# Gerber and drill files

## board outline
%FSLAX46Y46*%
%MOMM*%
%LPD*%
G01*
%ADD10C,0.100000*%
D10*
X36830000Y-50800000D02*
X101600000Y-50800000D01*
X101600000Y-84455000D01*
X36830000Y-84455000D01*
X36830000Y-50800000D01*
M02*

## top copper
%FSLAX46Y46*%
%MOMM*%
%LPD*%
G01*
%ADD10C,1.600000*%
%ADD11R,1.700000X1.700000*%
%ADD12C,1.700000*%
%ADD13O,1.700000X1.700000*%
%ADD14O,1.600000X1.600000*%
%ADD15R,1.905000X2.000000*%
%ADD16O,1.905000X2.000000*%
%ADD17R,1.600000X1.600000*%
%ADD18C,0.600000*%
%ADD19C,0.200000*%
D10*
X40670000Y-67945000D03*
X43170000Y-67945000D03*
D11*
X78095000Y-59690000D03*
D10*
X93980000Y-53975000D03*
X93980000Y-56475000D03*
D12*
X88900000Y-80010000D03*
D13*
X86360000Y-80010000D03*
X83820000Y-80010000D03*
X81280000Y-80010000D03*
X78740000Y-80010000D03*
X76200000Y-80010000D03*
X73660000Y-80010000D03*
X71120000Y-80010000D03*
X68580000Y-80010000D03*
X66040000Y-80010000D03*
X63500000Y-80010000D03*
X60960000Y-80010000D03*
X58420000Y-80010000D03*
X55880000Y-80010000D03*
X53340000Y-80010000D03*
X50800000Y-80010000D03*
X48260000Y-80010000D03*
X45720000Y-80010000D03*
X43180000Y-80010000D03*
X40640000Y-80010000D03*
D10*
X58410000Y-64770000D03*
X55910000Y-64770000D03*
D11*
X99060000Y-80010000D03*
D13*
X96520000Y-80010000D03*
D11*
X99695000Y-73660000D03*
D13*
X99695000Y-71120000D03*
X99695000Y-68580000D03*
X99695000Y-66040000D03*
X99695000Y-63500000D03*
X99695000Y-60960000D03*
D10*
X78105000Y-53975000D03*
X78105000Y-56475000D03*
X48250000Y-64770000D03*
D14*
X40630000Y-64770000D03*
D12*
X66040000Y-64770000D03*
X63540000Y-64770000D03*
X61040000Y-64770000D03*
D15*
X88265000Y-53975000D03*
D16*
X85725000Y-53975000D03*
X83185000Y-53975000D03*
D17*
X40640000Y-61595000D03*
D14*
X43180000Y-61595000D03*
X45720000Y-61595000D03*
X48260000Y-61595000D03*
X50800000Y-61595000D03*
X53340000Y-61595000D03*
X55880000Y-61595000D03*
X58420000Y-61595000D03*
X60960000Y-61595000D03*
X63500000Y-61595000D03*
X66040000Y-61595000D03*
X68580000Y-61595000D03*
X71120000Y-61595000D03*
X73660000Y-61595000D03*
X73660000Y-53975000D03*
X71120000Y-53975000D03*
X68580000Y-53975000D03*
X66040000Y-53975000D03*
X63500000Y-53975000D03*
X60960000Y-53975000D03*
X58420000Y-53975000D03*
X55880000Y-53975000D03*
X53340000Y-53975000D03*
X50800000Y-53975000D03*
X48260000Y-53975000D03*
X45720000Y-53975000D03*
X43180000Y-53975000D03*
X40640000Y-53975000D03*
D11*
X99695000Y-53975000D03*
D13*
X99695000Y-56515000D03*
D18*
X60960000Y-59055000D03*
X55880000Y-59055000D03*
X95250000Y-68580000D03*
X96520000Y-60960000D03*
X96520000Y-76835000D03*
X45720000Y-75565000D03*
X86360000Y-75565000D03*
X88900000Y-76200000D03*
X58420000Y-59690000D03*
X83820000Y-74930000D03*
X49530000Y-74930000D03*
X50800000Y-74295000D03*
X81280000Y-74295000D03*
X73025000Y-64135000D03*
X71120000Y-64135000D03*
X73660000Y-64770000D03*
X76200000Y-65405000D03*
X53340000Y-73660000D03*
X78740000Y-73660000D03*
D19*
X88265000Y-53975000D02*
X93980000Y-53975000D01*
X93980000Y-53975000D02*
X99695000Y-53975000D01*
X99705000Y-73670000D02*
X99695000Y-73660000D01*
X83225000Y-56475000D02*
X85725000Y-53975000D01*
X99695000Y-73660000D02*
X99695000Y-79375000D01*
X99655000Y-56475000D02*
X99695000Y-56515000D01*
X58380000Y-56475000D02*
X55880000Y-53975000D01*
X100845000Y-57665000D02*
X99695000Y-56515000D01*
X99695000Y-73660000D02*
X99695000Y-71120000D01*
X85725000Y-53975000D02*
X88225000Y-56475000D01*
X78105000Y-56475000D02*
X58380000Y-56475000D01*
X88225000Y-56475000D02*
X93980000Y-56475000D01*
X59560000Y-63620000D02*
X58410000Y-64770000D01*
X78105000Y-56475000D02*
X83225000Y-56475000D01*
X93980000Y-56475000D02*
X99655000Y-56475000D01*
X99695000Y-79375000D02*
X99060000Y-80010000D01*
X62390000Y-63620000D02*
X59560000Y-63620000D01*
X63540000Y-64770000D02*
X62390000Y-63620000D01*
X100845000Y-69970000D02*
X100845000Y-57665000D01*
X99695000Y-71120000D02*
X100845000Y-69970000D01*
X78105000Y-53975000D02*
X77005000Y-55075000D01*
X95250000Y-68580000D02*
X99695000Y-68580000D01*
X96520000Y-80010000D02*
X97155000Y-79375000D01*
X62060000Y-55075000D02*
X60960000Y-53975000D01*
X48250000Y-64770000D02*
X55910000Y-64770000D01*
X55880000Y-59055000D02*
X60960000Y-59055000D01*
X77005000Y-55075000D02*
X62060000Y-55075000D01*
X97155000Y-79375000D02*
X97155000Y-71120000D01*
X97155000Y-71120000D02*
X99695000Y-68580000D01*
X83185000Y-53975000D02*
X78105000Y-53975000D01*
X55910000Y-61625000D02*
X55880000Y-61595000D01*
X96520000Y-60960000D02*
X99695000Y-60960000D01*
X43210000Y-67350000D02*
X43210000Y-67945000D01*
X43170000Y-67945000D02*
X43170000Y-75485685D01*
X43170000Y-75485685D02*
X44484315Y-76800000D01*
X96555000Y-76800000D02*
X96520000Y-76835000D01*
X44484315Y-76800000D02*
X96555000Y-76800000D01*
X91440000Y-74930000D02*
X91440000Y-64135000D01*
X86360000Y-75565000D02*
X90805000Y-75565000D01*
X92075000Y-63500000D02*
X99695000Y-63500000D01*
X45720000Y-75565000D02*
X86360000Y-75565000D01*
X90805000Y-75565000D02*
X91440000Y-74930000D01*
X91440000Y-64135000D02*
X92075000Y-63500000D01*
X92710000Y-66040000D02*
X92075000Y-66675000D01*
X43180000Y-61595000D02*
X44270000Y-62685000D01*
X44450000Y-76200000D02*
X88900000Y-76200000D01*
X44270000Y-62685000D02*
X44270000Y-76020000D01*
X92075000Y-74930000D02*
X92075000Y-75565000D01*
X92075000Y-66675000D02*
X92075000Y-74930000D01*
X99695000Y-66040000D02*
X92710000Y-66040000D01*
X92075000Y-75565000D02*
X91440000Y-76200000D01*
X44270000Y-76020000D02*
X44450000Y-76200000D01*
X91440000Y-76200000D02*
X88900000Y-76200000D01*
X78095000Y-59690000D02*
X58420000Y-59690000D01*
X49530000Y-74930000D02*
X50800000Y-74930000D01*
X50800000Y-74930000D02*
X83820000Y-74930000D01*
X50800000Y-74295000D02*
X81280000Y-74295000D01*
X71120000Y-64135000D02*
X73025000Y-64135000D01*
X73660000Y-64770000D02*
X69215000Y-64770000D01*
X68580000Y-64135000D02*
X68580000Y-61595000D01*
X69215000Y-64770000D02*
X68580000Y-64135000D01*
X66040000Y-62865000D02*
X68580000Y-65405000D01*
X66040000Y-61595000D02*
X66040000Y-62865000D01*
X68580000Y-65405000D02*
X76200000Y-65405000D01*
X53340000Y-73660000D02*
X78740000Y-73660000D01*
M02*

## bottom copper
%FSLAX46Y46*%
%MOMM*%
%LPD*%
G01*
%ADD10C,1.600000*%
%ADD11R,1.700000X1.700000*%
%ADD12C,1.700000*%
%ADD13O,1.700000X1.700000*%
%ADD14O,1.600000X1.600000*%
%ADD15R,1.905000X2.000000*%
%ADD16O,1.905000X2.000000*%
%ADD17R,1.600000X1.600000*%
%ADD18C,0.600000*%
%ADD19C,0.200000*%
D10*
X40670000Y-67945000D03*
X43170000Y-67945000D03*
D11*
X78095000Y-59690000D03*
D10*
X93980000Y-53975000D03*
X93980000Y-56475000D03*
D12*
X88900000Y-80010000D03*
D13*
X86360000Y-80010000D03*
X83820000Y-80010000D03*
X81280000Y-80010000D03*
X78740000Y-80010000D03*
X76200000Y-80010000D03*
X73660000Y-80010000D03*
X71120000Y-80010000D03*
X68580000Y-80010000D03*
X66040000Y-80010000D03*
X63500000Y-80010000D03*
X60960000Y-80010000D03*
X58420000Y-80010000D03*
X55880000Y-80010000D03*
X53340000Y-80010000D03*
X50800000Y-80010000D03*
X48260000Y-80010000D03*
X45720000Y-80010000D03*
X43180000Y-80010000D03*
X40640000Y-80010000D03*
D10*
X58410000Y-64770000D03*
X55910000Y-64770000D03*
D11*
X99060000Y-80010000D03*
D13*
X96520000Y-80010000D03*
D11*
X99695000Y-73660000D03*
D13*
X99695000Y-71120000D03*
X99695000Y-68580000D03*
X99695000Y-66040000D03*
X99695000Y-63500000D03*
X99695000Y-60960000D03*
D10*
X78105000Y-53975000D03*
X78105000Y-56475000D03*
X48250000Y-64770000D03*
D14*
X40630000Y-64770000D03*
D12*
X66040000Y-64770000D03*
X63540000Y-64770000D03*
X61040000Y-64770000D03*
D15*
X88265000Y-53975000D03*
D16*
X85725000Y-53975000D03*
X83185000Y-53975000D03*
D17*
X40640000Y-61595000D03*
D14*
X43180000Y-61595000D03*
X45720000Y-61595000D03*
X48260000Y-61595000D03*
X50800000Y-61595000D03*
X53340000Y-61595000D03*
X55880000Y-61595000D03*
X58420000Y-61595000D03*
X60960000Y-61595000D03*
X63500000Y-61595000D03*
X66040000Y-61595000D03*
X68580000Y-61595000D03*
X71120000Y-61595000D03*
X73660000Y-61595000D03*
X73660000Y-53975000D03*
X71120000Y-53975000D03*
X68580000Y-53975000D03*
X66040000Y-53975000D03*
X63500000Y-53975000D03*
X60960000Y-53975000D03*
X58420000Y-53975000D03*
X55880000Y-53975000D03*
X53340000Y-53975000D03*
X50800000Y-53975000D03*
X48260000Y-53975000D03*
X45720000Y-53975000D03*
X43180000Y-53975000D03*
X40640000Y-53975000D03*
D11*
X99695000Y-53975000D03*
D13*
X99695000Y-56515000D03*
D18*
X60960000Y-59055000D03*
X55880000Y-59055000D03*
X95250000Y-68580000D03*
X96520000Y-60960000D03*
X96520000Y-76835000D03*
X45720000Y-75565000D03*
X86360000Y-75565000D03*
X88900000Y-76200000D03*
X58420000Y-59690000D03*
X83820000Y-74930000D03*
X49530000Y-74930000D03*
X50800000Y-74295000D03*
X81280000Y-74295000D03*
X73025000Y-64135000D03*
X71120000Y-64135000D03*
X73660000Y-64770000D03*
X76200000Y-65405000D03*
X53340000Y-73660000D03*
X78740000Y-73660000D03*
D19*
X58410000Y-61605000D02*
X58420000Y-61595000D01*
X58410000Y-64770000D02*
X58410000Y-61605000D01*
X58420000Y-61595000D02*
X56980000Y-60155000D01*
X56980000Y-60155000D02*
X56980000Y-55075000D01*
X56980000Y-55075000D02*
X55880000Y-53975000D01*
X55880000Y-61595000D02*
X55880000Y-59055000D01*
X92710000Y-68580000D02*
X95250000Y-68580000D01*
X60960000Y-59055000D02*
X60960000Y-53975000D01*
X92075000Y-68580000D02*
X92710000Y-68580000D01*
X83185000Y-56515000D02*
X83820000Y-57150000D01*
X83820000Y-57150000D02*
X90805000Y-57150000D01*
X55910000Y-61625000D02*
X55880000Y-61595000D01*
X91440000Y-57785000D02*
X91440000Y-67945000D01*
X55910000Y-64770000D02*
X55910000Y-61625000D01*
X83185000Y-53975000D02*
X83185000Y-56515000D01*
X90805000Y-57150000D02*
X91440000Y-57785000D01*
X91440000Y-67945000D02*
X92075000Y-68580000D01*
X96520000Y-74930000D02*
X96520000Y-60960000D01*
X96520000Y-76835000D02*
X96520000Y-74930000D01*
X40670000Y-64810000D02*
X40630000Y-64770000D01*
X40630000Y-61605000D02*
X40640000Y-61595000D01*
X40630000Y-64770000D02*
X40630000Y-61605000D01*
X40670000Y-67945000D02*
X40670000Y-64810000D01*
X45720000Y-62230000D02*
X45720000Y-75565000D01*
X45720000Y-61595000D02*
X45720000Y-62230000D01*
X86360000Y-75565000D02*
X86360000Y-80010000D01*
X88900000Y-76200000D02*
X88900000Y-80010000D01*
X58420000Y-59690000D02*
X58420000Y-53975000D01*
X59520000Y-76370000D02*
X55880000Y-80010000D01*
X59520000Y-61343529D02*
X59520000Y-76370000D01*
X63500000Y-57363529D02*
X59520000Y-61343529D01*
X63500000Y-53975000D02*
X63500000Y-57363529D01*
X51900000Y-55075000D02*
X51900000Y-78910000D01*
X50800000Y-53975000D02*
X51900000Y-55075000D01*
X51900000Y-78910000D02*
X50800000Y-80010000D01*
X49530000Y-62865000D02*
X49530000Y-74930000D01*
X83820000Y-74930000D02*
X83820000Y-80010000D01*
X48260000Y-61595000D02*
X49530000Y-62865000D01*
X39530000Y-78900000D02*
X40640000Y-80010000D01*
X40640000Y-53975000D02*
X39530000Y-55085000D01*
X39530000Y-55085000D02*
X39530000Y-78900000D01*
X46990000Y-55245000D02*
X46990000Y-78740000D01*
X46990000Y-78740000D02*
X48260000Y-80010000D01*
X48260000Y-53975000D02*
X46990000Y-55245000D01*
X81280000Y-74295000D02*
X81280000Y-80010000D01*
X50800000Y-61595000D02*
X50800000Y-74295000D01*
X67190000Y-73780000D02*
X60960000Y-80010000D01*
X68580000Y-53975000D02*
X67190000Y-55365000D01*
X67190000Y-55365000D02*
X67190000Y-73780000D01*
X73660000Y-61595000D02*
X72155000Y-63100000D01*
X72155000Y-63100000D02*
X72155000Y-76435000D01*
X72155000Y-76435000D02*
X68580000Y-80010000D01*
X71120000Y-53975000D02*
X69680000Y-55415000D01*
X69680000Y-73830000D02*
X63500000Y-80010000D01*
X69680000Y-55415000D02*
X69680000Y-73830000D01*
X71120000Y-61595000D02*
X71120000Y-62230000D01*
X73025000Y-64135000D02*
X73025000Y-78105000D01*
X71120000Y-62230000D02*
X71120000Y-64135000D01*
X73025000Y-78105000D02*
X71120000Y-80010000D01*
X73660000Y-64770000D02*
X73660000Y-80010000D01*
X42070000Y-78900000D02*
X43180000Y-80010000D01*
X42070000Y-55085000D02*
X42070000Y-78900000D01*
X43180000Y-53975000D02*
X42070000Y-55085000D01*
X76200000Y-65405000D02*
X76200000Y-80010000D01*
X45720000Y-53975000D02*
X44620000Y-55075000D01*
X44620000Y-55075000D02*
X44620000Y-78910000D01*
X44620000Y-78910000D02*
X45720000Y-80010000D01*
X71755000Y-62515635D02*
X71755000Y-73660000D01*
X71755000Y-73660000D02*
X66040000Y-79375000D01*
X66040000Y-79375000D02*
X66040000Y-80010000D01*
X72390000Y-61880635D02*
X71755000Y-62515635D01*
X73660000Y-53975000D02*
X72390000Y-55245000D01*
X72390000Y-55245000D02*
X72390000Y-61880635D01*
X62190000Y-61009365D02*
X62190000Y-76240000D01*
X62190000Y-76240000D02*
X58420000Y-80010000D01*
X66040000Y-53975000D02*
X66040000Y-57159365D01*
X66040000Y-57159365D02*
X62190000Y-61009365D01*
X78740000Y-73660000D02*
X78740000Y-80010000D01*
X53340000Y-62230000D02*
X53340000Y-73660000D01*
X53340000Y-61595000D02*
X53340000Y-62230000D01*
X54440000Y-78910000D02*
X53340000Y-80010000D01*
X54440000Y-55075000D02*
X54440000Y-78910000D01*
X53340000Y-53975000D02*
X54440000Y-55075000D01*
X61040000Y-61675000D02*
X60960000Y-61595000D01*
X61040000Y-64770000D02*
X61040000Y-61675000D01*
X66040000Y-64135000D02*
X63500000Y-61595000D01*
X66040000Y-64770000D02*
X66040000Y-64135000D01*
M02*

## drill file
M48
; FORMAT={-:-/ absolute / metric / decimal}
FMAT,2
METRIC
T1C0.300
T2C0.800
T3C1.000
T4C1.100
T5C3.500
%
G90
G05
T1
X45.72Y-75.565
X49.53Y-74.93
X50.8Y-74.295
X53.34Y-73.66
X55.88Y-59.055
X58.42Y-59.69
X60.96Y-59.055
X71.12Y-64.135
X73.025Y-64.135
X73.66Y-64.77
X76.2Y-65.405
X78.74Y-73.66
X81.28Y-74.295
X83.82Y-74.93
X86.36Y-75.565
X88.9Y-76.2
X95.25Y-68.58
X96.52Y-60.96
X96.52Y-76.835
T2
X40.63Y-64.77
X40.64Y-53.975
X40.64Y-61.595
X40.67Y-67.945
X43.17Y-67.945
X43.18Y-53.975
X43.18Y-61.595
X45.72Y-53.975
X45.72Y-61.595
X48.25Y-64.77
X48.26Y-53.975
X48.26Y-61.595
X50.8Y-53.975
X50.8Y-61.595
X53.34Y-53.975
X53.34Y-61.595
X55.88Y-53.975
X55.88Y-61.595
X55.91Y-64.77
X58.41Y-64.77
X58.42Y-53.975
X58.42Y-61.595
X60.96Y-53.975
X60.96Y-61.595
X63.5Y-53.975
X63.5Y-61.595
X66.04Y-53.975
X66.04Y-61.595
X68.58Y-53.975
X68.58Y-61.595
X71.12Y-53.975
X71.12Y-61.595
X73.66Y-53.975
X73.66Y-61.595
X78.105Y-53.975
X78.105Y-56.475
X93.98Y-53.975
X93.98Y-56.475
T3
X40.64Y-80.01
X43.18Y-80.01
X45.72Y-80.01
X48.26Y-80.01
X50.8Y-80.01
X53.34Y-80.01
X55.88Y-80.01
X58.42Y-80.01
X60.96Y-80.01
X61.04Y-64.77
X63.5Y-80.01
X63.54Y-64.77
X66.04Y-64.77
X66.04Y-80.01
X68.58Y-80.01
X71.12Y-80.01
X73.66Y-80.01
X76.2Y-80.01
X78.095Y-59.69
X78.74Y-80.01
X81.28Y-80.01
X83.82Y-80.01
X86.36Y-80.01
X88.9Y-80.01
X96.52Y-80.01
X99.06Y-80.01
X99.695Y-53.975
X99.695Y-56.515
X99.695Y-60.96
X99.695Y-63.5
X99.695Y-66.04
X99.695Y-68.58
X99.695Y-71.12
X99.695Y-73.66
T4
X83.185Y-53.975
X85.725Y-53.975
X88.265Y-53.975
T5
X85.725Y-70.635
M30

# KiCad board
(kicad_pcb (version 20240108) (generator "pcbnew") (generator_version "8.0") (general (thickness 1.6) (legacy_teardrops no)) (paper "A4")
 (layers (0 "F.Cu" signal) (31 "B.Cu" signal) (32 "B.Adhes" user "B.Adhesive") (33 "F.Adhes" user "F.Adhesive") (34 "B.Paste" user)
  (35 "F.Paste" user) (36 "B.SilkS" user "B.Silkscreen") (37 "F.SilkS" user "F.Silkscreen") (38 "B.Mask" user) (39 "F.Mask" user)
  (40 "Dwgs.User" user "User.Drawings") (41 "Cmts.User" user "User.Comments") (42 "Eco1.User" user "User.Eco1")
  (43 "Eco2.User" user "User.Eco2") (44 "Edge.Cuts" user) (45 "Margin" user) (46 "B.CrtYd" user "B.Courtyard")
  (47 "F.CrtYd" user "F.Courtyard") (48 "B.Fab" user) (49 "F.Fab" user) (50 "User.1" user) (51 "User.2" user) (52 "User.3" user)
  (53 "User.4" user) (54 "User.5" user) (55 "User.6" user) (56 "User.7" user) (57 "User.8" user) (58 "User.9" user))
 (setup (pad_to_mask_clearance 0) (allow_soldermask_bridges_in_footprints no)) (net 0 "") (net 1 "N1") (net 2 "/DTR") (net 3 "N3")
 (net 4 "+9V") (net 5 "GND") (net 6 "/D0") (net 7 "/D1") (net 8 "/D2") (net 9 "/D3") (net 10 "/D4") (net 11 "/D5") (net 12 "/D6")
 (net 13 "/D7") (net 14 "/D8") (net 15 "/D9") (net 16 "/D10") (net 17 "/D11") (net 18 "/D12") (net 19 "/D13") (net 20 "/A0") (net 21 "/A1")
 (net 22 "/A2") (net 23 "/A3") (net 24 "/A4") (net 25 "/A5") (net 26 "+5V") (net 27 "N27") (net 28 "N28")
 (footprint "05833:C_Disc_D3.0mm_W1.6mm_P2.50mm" (layer "F.Cu") (at 40.67 67.945)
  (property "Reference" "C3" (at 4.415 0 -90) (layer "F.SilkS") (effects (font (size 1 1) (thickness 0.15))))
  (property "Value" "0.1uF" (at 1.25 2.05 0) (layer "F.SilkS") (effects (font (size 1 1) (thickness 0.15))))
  (pad "1" thru_hole circle (at 0 0) (size 1.6 1.6) (drill 0.8) (layers "*.Cu" "*.Mask") (remove_unused_layers no) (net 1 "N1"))
  (pad "2" thru_hole circle (at 2.5 0) (size 1.6 1.6) (drill 0.8) (layers "*.Cu" "*.Mask") (remove_unused_layers no) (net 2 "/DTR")))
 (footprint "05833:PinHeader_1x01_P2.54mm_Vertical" (layer "F.Cu") (at 78.095 59.69)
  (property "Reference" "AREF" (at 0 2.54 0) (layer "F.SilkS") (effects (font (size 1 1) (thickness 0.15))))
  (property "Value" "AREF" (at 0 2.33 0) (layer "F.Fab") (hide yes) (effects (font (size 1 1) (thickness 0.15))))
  (pad "1" thru_hole rect (at 0 0) (size 1.7 1.7) (drill 1) (layers "*.Cu" "*.Mask") (remove_unused_layers no) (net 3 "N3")))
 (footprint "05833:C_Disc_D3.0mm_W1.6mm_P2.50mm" (layer "F.Cu") (at 93.98 53.975 -90)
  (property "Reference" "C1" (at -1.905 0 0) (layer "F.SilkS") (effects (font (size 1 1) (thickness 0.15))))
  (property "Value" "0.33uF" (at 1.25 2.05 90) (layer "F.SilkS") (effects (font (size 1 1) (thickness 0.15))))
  (pad "1" thru_hole circle (at 0 0 270) (size 1.6 1.6) (drill 0.8) (layers "*.Cu" "*.Mask") (remove_unused_layers no) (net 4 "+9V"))
  (pad "2" thru_hole circle (at 2.5 0 270) (size 1.6 1.6) (drill 0.8) (layers "*.Cu" "*.Mask") (remove_unused_layers no) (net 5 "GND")))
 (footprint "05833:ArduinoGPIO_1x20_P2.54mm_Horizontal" (layer "F.Cu") (at 88.9 80.01 -90)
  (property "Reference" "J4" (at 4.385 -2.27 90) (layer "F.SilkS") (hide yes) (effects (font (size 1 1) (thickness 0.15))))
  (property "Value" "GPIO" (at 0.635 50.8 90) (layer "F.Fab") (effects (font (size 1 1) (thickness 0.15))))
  (pad "1" thru_hole circle (at 0 0 270) (size 1.7 1.7) (drill 1) (layers "*.Cu" "*.Mask") (remove_unused_layers no) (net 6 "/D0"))
  (pad "2" thru_hole oval (at 0 2.54 270) (size 1.7 1.7) (drill 1) (layers "*.Cu" "*.Mask") (remove_unused_layers no) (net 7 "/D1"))
  (pad "3" thru_hole oval (at 0 5.08 270) (size 1.7 1.7) (drill 1) (layers "*.Cu" "*.Mask") (remove_unused_layers no) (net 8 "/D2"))
  (pad "4" thru_hole oval (at 0 7.62 270) (size 1.7 1.7) (drill 1) (layers "*.Cu" "*.Mask") (remove_unused_layers no) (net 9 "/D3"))
  (pad "5" thru_hole oval (at 0 10.16 270) (size 1.7 1.7) (drill 1) (layers "*.Cu" "*.Mask") (remove_unused_layers no) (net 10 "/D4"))
  (pad "6" thru_hole oval (at 0 12.7 270) (size 1.7 1.7) (drill 1) (layers "*.Cu" "*.Mask") (remove_unused_layers no) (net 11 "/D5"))
  (pad "7" thru_hole oval (at 0 15.24 270) (size 1.7 1.7) (drill 1) (layers "*.Cu" "*.Mask") (remove_unused_layers no) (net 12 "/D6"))
  (pad "8" thru_hole oval (at 0 17.78 270) (size 1.7 1.7) (drill 1) (layers "*.Cu" "*.Mask") (remove_unused_layers no) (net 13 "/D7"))
  (pad "9" thru_hole oval (at 0 20.32 270) (size 1.7 1.7) (drill 1) (layers "*.Cu" "*.Mask") (remove_unused_layers no) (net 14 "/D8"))
  (pad "10" thru_hole oval (at 0 22.86 270) (size 1.7 1.7) (drill 1) (layers "*.Cu" "*.Mask") (remove_unused_layers no) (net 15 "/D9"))
  (pad "11" thru_hole oval (at 0 25.4 270) (size 1.7 1.7) (drill 1) (layers "*.Cu" "*.Mask") (remove_unused_layers no) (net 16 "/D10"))
  (pad "12" thru_hole oval (at 0 27.94 270) (size 1.7 1.7) (drill 1) (layers "*.Cu" "*.Mask") (remove_unused_layers no) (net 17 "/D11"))
  (pad "13" thru_hole oval (at 0 30.48 270) (size 1.7 1.7) (drill 1) (layers "*.Cu" "*.Mask") (remove_unused_layers no) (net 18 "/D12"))
  (pad "14" thru_hole oval (at 0 33.02 270) (size 1.7 1.7) (drill 1) (layers "*.Cu" "*.Mask") (remove_unused_layers no) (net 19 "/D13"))
  (pad "15" thru_hole oval (at 0 35.56 270) (size 1.7 1.7) (drill 1) (layers "*.Cu" "*.Mask") (remove_unused_layers no) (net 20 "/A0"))
  (pad "16" thru_hole oval (at 0 38.1 270) (size 1.7 1.7) (drill 1) (layers "*.Cu" "*.Mask") (remove_unused_layers no) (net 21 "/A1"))
  (pad "17" thru_hole oval (at 0 40.64 270) (size 1.7 1.7) (drill 1) (layers "*.Cu" "*.Mask") (remove_unused_layers no) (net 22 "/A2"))
  (pad "18" thru_hole oval (at 0 43.18 270) (size 1.7 1.7) (drill 1) (layers "*.Cu" "*.Mask") (remove_unused_layers no) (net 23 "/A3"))
  (pad "19" thru_hole oval (at 0 45.72 270) (size 1.7 1.7) (drill 1) (layers "*.Cu" "*.Mask") (remove_unused_layers no) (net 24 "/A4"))
  (pad "20" thru_hole oval (at 0 48.26 270) (size 1.7 1.7) (drill 1) (layers "*.Cu" "*.Mask") (remove_unused_layers no) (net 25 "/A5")))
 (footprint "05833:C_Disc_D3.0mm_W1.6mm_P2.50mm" (layer "F.Cu") (at 58.41 64.77 180)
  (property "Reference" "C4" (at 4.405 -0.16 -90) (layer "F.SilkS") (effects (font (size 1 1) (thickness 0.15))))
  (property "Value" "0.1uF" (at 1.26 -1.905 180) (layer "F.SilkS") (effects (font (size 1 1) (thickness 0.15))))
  (pad "1" thru_hole circle (at 0 0 180) (size 1.6 1.6) (drill 0.8) (layers "*.Cu" "*.Mask") (remove_unused_layers no) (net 5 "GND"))
  (pad "2" thru_hole circle (at 2.5 0 180) (size 1.6 1.6) (drill 0.8) (layers "*.Cu" "*.Mask") (remove_unused_layers no) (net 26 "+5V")))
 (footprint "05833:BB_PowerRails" (layer "F.Cu") (at 99.06 80.01 -90)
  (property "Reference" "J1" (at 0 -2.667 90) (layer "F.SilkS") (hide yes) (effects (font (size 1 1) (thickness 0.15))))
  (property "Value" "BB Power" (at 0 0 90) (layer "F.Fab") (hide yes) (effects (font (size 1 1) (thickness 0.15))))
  (pad "1" thru_hole rect (at 0 0 270) (size 1.7 1.7) (drill 1) (layers "*.Cu" "*.Mask") (remove_unused_layers no) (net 5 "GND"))
  (pad "2" thru_hole oval (at 0 2.54 270) (size 1.7 1.7) (drill 1) (layers "*.Cu" "*.Mask") (remove_unused_layers no) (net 26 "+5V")))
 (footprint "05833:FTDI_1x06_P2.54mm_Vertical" (layer "F.Cu") (at 99.695 73.66 180)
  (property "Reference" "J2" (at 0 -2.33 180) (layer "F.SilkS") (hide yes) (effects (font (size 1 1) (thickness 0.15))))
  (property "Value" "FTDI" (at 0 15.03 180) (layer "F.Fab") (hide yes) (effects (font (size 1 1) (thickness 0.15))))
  (pad "1" thru_hole rect (at 0 0 180) (size 1.7 1.7) (drill 1) (layers "*.Cu" "*.Mask") (remove_unused_layers no) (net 5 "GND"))
  (pad "2" thru_hole oval (at 0 2.54 180) (size 1.7 1.7) (drill 1) (layers "*.Cu" "*.Mask") (remove_unused_layers no) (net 5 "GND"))
  (pad "3" thru_hole oval (at 0 5.08 180) (size 1.7 1.7) (drill 1) (layers "*.Cu" "*.Mask") (remove_unused_layers no) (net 26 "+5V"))
  (pad "4" thru_hole oval (at 0 7.62 180) (size 1.7 1.7) (drill 1) (layers "*.Cu" "*.Mask") (remove_unused_layers no) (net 6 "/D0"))
  (pad "5" thru_hole oval (at 0 10.16 180) (size 1.7 1.7) (drill 1) (layers "*.Cu" "*.Mask") (remove_unused_layers no) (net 7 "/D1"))
  (pad "6" thru_hole oval (at 0 12.7 180) (size 1.7 1.7) (drill 1) (layers "*.Cu" "*.Mask") (remove_unused_layers no) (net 2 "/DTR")))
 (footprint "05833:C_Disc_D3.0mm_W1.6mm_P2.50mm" (layer "F.Cu") (at 78.105 53.975 -90)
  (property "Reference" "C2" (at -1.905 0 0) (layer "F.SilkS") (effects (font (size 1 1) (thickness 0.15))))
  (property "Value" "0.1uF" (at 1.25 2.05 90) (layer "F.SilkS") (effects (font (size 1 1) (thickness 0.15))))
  (pad "1" thru_hole circle (at 0 0 270) (size 1.6 1.6) (drill 0.8) (layers "*.Cu" "*.Mask") (remove_unused_layers no) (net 26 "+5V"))
  (pad "2" thru_hole circle (at 2.5 0 270) (size 1.6 1.6) (drill 0.8) (layers "*.Cu" "*.Mask") (remove_unused_layers no) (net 5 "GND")))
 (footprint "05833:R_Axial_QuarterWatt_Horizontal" (layer "F.Cu") (at 48.25 64.77 180)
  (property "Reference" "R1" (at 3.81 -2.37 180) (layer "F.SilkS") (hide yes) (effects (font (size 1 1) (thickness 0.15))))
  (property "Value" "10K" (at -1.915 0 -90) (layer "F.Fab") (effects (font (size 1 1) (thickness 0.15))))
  (pad "1" thru_hole circle (at 0 0 180) (size 1.6 1.6) (drill 0.8) (layers "*.Cu" "*.Mask") (remove_unused_layers no) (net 26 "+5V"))
  (pad "2" thru_hole oval (at 7.62 0 180) (size 1.6 1.6) (drill 0.8) (layers "*.Cu" "*.Mask") (remove_unused_layers no) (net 1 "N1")))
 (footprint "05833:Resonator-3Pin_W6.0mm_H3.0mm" (layer "F.Cu") (at 66.04 64.77 180)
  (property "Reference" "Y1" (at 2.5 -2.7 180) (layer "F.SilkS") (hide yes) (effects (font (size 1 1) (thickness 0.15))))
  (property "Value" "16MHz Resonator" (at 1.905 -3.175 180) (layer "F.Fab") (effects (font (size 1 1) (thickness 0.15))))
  (pad "1" thru_hole circle (at 0 0 180) (size 1.7 1.7) (drill 1) (layers "*.Cu" "*.Mask") (remove_unused_layers no) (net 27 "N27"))
  (pad "2" thru_hole circle (at 2.5 0 180) (size 1.7 1.7) (drill 1) (layers "*.Cu" "*.Mask") (remove_unused_layers no) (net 5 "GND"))
  (pad "3" thru_hole circle (at 5 0 180) (size 1.7 1.7) (drill 1) (layers "*.Cu" "*.Mask") (remove_unused_layers no) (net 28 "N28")))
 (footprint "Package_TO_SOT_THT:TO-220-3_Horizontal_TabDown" (layer "F.Cu") (at 88.265 53.975 180)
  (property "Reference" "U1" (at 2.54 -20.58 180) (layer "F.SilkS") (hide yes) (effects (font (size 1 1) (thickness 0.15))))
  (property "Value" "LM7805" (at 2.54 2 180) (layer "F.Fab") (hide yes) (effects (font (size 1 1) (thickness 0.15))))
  (pad "" np_thru_hole oval (at 2.54 -16.66 180) (size 3.5 3.5) (drill 3.5) (layers "*.Cu" "*.Mask"))
  (pad "1" thru_hole rect (at 0 0 180) (size 1.905 2) (drill 1.1) (layers "*.Cu" "*.Mask") (remove_unused_layers no) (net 4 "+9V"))
  (pad "2" thru_hole oval (at 2.54 0 180) (size 1.905 2) (drill 1.1) (layers "*.Cu" "*.Mask") (remove_unused_layers no) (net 5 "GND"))
  (pad "3" thru_hole oval (at 5.08 0 180) (size 1.905 2) (drill 1.1) (layers "*.Cu" "*.Mask") (remove_unused_layers no) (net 26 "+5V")))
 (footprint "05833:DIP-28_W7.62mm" (layer "F.Cu") (at 40.64 61.595 90)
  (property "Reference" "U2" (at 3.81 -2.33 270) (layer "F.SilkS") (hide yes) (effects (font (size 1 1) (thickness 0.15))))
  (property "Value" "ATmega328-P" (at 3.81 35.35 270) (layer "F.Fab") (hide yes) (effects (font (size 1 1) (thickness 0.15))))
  (pad "1" thru_hole rect (at 0 0 90) (size 1.6 1.6) (drill 0.8) (layers "*.Cu" "*.Mask") (remove_unused_layers no) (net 1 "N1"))
  (pad "2" thru_hole oval (at 0 2.54 90) (size 1.6 1.6) (drill 0.8) (layers "*.Cu" "*.Mask") (remove_unused_layers no) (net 6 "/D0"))
  (pad "3" thru_hole oval (at 0 5.08 90) (size 1.6 1.6) (drill 0.8) (layers "*.Cu" "*.Mask") (remove_unused_layers no) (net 7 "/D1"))
  (pad "4" thru_hole oval (at 0 7.62 90) (size 1.6 1.6) (drill 0.8) (layers "*.Cu" "*.Mask") (remove_unused_layers no) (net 8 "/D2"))
  (pad "5" thru_hole oval (at 0 10.16 90) (size 1.6 1.6) (drill 0.8) (layers "*.Cu" "*.Mask") (remove_unused_layers no) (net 9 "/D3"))
  (pad "6" thru_hole oval (at 0 12.7 90) (size 1.6 1.6) (drill 0.8) (layers "*.Cu" "*.Mask") (remove_unused_layers no) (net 10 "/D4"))
  (pad "7" thru_hole oval (at 0 15.24 90) (size 1.6 1.6) (drill 0.8) (layers "*.Cu" "*.Mask") (remove_unused_layers no) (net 26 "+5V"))
  (pad "8" thru_hole oval (at 0 17.78 90) (size 1.6 1.6) (drill 0.8) (layers "*.Cu" "*.Mask") (remove_unused_layers no) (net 5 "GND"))
  (pad "9" thru_hole oval (at 0 20.32 90) (size 1.6 1.6) (drill 0.8) (layers "*.Cu" "*.Mask") (remove_unused_layers no) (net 28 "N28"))
  (pad "10" thru_hole oval (at 0 22.86 90) (size 1.6 1.6) (drill 0.8) (layers "*.Cu" "*.Mask") (remove_unused_layers no) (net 27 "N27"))
  (pad "11" thru_hole oval (at 0 25.4 90) (size 1.6 1.6) (drill 0.8) (layers "*.Cu" "*.Mask") (remove_unused_layers no) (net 11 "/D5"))
  (pad "12" thru_hole oval (at 0 27.94 90) (size 1.6 1.6) (drill 0.8) (layers "*.Cu" "*.Mask") (remove_unused_layers no) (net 12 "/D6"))
  (pad "13" thru_hole oval (at 0 30.48 90) (size 1.6 1.6) (drill 0.8) (layers "*.Cu" "*.Mask") (remove_unused_layers no) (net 13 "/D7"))
  (pad "14" thru_hole oval (at 0 33.02 90) (size 1.6 1.6) (drill 0.8) (layers "*.Cu" "*.Mask") (remove_unused_layers no) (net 14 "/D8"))
  (pad "15" thru_hole oval (at 7.62 33.02 90) (size 1.6 1.6) (drill 0.8) (layers "*.Cu" "*.Mask") (remove_unused_layers no) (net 15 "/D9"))
  (pad "16" thru_hole oval (at 7.62 30.48 90) (size 1.6 1.6) (drill 0.8) (layers "*.Cu" "*.Mask") (remove_unused_layers no) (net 16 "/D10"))
  (pad "17" thru_hole oval (at 7.62 27.94 90) (size 1.6 1.6) (drill 0.8) (layers "*.Cu" "*.Mask") (remove_unused_layers no) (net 17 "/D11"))
  (pad "18" thru_hole oval (at 7.62 25.4 90) (size 1.6 1.6) (drill 0.8) (layers "*.Cu" "*.Mask") (remove_unused_layers no) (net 18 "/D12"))
  (pad "19" thru_hole oval (at 7.62 22.86 90) (size 1.6 1.6) (drill 0.8) (layers "*.Cu" "*.Mask") (remove_unused_layers no) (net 19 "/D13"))
  (pad "20" thru_hole oval (at 7.62 20.32 90) (size 1.6 1.6) (drill 0.8) (layers "*.Cu" "*.Mask") (remove_unused_layers no) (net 26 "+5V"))
  (pad "21" thru_hole oval (at 7.62 17.78 90) (size 1.6 1.6) (drill 0.8) (layers "*.Cu" "*.Mask") (remove_unused_layers no) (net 3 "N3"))
  (pad "22" thru_hole oval (at 7.62 15.24 90) (size 1.6 1.6) (drill 0.8) (layers "*.Cu" "*.Mask") (remove_unused_layers no) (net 5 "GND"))
  (pad "23" thru_hole oval (at 7.62 12.7 90) (size 1.6 1.6) (drill 0.8) (layers "*.Cu" "*.Mask") (remove_unused_layers no) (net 20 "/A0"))
  (pad "24" thru_hole oval (at 7.62 10.16 90) (size 1.6 1.6) (drill 0.8) (layers "*.Cu" "*.Mask") (remove_unused_layers no) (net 21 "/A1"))
  (pad "25" thru_hole oval (at 7.62 7.62 90) (size 1.6 1.6) (drill 0.8) (layers "*.Cu" "*.Mask") (remove_unused_layers no) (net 22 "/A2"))
  (pad "26" thru_hole oval (at 7.62 5.08 90) (size 1.6 1.6) (drill 0.8) (layers "*.Cu" "*.Mask") (remove_unused_layers no) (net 23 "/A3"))
  (pad "27" thru_hole oval (at 7.62 2.54 90) (size 1.6 1.6) (drill 0.8) (layers "*.Cu" "*.Mask") (remove_unused_layers no) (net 24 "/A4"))
  (pad "28" thru_hole oval (at 7.62 0 90) (size 1.6 1.6) (drill 0.8) (layers "*.Cu" "*.Mask") (remove_unused_layers no) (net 25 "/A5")))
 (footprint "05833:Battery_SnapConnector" (layer "F.Cu") (at 99.695 53.975)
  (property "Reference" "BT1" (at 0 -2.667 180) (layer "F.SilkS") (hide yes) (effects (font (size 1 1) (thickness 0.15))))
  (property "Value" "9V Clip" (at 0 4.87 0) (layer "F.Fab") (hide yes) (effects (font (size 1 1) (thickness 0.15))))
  (pad "1" thru_hole rect (at 0 0) (size 1.7 1.7) (drill 1) (layers "*.Cu" "*.Mask") (remove_unused_layers no) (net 4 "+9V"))
  (pad "2" thru_hole oval (at 0 2.54) (size 1.7 1.7) (drill 1) (layers "*.Cu" "*.Mask") (remove_unused_layers no) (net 5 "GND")))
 (gr_rect (start 36.83 50.8) (end 101.6 84.455) (stroke (width 0.1) (type default)) (fill none) (layer "Edge.Cuts"))
 (segment (start 88.265 53.975) (end 93.98 53.975) (width 0.2) (layer "F.Cu") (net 4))
 (segment (start 93.98 53.975) (end 99.695 53.975) (width 0.2) (layer "F.Cu") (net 4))
 (segment (start 99.705 73.67) (end 99.695 73.66) (width 0.2) (layer "F.Cu") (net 5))
 (segment (start 83.225 56.475) (end 85.725 53.975) (width 0.2) (layer "F.Cu") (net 5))
 (segment (start 99.695 73.66) (end 99.695 79.375) (width 0.2) (layer "F.Cu") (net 5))
 (segment (start 99.655 56.475) (end 99.695 56.515) (width 0.2) (layer "F.Cu") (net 5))
 (segment (start 58.38 56.475) (end 55.88 53.975) (width 0.2) (layer "F.Cu") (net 5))
 (segment (start 100.845 57.665) (end 99.695 56.515) (width 0.2) (layer "F.Cu") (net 5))
 (segment (start 99.695 73.66) (end 99.695 71.12) (width 0.2) (layer "F.Cu") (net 5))
 (segment (start 85.725 53.975) (end 88.225 56.475) (width 0.2) (layer "F.Cu") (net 5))
 (segment (start 78.105 56.475) (end 58.38 56.475) (width 0.2) (layer "F.Cu") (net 5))
 (segment (start 88.225 56.475) (end 93.98 56.475) (width 0.2) (layer "F.Cu") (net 5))
 (segment (start 59.56 63.62) (end 58.41 64.77) (width 0.2) (layer "F.Cu") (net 5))
 (segment (start 78.105 56.475) (end 83.225 56.475) (width 0.2) (layer "F.Cu") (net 5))
 (segment (start 93.98 56.475) (end 99.655 56.475) (width 0.2) (layer "F.Cu") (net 5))
 (segment (start 99.695 79.375) (end 99.06 80.01) (width 0.2) (layer "F.Cu") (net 5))
 (segment (start 62.39 63.62) (end 59.56 63.62) (width 0.2) (layer "F.Cu") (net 5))
 (segment (start 63.54 64.77) (end 62.39 63.62) (width 0.2) (layer "F.Cu") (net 5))
 (segment (start 100.845 69.97) (end 100.845 57.665) (width 0.2) (layer "F.Cu") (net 5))
 (segment (start 99.695 71.12) (end 100.845 69.97) (width 0.2) (layer "F.Cu") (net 5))
 (segment (start 58.41 61.605) (end 58.42 61.595) (width 0.2) (layer "B.Cu") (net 5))
 (segment (start 58.41 64.77) (end 58.41 61.605) (width 0.2) (layer "B.Cu") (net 5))
 (segment (start 58.42 61.595) (end 56.98 60.155) (width 0.2) (layer "B.Cu") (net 5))
 (segment (start 56.98 60.155) (end 56.98 55.075) (width 0.2) (layer "B.Cu") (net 5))
 (segment (start 56.98 55.075) (end 55.88 53.975) (width 0.2) (layer "B.Cu") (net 5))
 (segment (start 78.105 53.975) (end 77.005 55.075) (width 0.2) (layer "F.Cu") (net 26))
 (segment (start 95.25 68.58) (end 99.695 68.58) (width 0.2) (layer "F.Cu") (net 26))
 (segment (start 96.52 80.01) (end 97.155 79.375) (width 0.2) (layer "F.Cu") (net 26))
 (segment (start 62.06 55.075) (end 60.96 53.975) (width 0.2) (layer "F.Cu") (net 26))
 (segment (start 48.25 64.77) (end 55.91 64.77) (width 0.2) (layer "F.Cu") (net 26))
 (segment (start 55.88 59.055) (end 60.96 59.055) (width 0.2) (layer "F.Cu") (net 26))
 (segment (start 77.005 55.075) (end 62.06 55.075) (width 0.2) (layer "F.Cu") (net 26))
 (segment (start 97.155 79.375) (end 97.155 71.12) (width 0.2) (layer "F.Cu") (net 26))
 (segment (start 97.155 71.12) (end 99.695 68.58) (width 0.2) (layer "F.Cu") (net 26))
 (segment (start 83.185 53.975) (end 78.105 53.975) (width 0.2) (layer "F.Cu") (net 26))
 (segment (start 55.91 61.625) (end 55.88 61.595) (width 0.2) (layer "F.Cu") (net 26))
 (via (at 60.96 59.055) (size 0.6) (drill 0.3) (layers "F.Cu" "B.Cu") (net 26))
 (via (at 55.88 59.055) (size 0.6) (drill 0.3) (layers "F.Cu" "B.Cu") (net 26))
 (via (at 95.25 68.58) (size 0.6) (drill 0.3) (layers "F.Cu" "B.Cu") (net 26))
 (segment (start 55.88 61.595) (end 55.88 59.055) (width 0.2) (layer "B.Cu") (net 26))
 (segment (start 92.71 68.58) (end 95.25 68.58) (width 0.2) (layer "B.Cu") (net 26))
 (segment (start 60.96 59.055) (end 60.96 53.975) (width 0.2) (layer "B.Cu") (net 26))
 (segment (start 92.075 68.58) (end 92.71 68.58) (width 0.2) (layer "B.Cu") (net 26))
 (segment (start 83.185 56.515) (end 83.82 57.15) (width 0.2) (layer "B.Cu") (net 26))
 (segment (start 83.82 57.15) (end 90.805 57.15) (width 0.2) (layer "B.Cu") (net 26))
 (segment (start 55.91 61.625) (end 55.88 61.595) (width 0.2) (layer "B.Cu") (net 26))
 (segment (start 91.44 57.785) (end 91.44 67.945) (width 0.2) (layer "B.Cu") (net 26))
 (segment (start 55.91 64.77) (end 55.91 61.625) (width 0.2) (layer "B.Cu") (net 26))
 (segment (start 83.185 53.975) (end 83.185 56.515) (width 0.2) (layer "B.Cu") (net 26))
 (segment (start 90.805 57.15) (end 91.44 57.785) (width 0.2) (layer "B.Cu") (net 26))
 (segment (start 91.44 67.945) (end 92.075 68.58) (width 0.2) (layer "B.Cu") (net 26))
 (segment (start 96.52 60.96) (end 99.695 60.96) (width 0.2) (layer "F.Cu") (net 2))
 (segment (start 43.21 67.35) (end 43.21 67.945) (width 0.2) (layer "F.Cu") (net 2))
 (segment (start 43.17 67.945) (end 43.17 75.485685) (width 0.2) (layer "F.Cu") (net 2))
 (segment (start 43.17 75.485685) (end 44.484315 76.8) (width 0.2) (layer "F.Cu") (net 2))
 (segment (start 96.555 76.8) (end 96.52 76.835) (width 0.2) (layer "F.Cu") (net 2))
 (segment (start 44.484315 76.8) (end 96.555 76.8) (width 0.2) (layer "F.Cu") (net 2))
 (via (at 96.52 60.96) (size 0.6) (drill 0.3) (layers "F.Cu" "B.Cu") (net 2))
 (via (at 96.52 76.835) (size 0.6) (drill 0.3) (layers "F.Cu" "B.Cu") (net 2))
 (segment (start 96.52 74.93) (end 96.52 60.96) (width 0.2) (layer "B.Cu") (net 2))
 (segment (start 96.52 76.835) (end 96.52 74.93) (width 0.2) (layer "B.Cu") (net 2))
 (segment (start 40.67 64.81) (end 40.63 64.77) (width 0.2) (layer "B.Cu") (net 1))
 (segment (start 40.63 61.605) (end 40.64 61.595) (width 0.2) (layer "B.Cu") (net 1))
 (segment (start 40.63 64.77) (end 40.63 61.605) (width 0.2) (layer "B.Cu") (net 1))
 (segment (start 40.67 67.945) (end 40.67 64.81) (width 0.2) (layer "B.Cu") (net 1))
 (segment (start 91.44 74.93) (end 91.44 64.135) (width 0.2) (layer "F.Cu") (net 7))
 (segment (start 86.36 75.565) (end 90.805 75.565) (width 0.2) (layer "F.Cu") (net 7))
 (segment (start 92.075 63.5) (end 99.695 63.5) (width 0.2) (layer "F.Cu") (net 7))
 (segment (start 45.72 75.565) (end 86.36 75.565) (width 0.2) (layer "F.Cu") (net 7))
 (segment (start 90.805 75.565) (end 91.44 74.93) (width 0.2) (layer "F.Cu") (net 7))
 (segment (start 91.44 64.135) (end 92.075 63.5) (width 0.2) (layer "F.Cu") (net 7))
 (via (at 45.72 75.565) (size 0.6) (drill 0.3) (layers "F.Cu" "B.Cu") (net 7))
 (via (at 86.36 75.565) (size 0.6) (drill 0.3) (layers "F.Cu" "B.Cu") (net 7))
 (segment (start 45.72 62.23) (end 45.72 75.565) (width 0.2) (layer "B.Cu") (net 7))
 (segment (start 45.72 61.595) (end 45.72 62.23) (width 0.2) (layer "B.Cu") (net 7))
 (segment (start 86.36 75.565) (end 86.36 80.01) (width 0.2) (layer "B.Cu") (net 7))
 (segment (start 92.71 66.04) (end 92.075 66.675) (width 0.2) (layer "F.Cu") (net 6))
 (segment (start 43.18 61.595) (end 44.27 62.685) (width 0.2) (layer "F.Cu") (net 6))
 (segment (start 44.45 76.2) (end 88.9 76.2) (width 0.2) (layer "F.Cu") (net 6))
 (segment (start 44.27 62.685) (end 44.27 76.02) (width 0.2) (layer "F.Cu") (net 6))
 (segment (start 92.075 74.93) (end 92.075 75.565) (width 0.2) (layer "F.Cu") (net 6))
 (segment (start 92.075 66.675) (end 92.075 74.93) (width 0.2) (layer "F.Cu") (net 6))
 (segment (start 99.695 66.04) (end 92.71 66.04) (width 0.2) (layer "F.Cu") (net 6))
 (segment (start 92.075 75.565) (end 91.44 76.2) (width 0.2) (layer "F.Cu") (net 6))
 (segment (start 44.27 76.02) (end 44.45 76.2) (width 0.2) (layer "F.Cu") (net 6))
 (segment (start 91.44 76.2) (end 88.9 76.2) (width 0.2) (layer "F.Cu") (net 6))
 (via (at 88.9 76.2) (size 0.6) (drill 0.3) (layers "F.Cu" "B.Cu") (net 6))
 (segment (start 88.9 76.2) (end 88.9 80.01) (width 0.2) (layer "B.Cu") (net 6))
 (segment (start 78.095 59.69) (end 58.42 59.69) (width 0.2) (layer "F.Cu") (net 3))
 (via (at 58.42 59.69) (size 0.6) (drill 0.3) (layers "F.Cu" "B.Cu") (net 3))
 (segment (start 58.42 59.69) (end 58.42 53.975) (width 0.2) (layer "B.Cu") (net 3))
 (segment (start 59.52 76.37) (end 55.88 80.01) (width 0.2) (layer "B.Cu") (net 19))
 (segment (start 59.52 61.343529) (end 59.52 76.37) (width 0.2) (layer "B.Cu") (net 19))
 (segment (start 63.5 57.363529) (end 59.52 61.343529) (width 0.2) (layer "B.Cu") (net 19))
 (segment (start 63.5 53.975) (end 63.5 57.363529) (width 0.2) (layer "B.Cu") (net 19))
 (segment (start 51.9 55.075) (end 51.9 78.91) (width 0.2) (layer "B.Cu") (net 21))
 (segment (start 50.8 53.975) (end 51.9 55.075) (width 0.2) (layer "B.Cu") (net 21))
 (segment (start 51.9 78.91) (end 50.8 80.01) (width 0.2) (layer "B.Cu") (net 21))
 (segment (start 49.53 74.93) (end 50.8 74.93) (width 0.2) (layer "F.Cu") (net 8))
 (segment (start 50.8 74.93) (end 83.82 74.93) (width 0.2) (layer "F.Cu") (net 8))
 (via (at 83.82 74.93) (size 0.6) (drill 0.3) (layers "F.Cu" "B.Cu") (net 8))
 (via (at 49.53 74.93) (size 0.6) (drill 0.3) (layers "F.Cu" "B.Cu") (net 8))
 (segment (start 49.53 62.865) (end 49.53 74.93) (width 0.2) (layer "B.Cu") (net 8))
 (segment (start 83.82 74.93) (end 83.82 80.01) (width 0.2) (layer "B.Cu") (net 8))
 (segment (start 48.26 61.595) (end 49.53 62.865) (width 0.2) (layer "B.Cu") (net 8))
 (segment (start 39.53 78.9) (end 40.64 80.01) (width 0.2) (layer "B.Cu") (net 25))
 (segment (start 40.64 53.975) (end 39.53 55.085) (width 0.2) (layer "B.Cu") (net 25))
 (segment (start 39.53 55.085) (end 39.53 78.9) (width 0.2) (layer "B.Cu") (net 25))
 (segment (start 46.99 55.245) (end 46.99 78.74) (width 0.2) (layer "B.Cu") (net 22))
 (segment (start 46.99 78.74) (end 48.26 80.01) (width 0.2) (layer "B.Cu") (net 22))
 (segment (start 48.26 53.975) (end 46.99 55.245) (width 0.2) (layer "B.Cu") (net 22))
 (segment (start 50.8 74.295) (end 81.28 74.295) (width 0.2) (layer "F.Cu") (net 9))
 (via (at 50.8 74.295) (size 0.6) (drill 0.3) (layers "F.Cu" "B.Cu") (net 9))
 (via (at 81.28 74.295) (size 0.6) (drill 0.3) (layers "F.Cu" "B.Cu") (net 9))
 (segment (start 81.28 74.295) (end 81.28 80.01) (width 0.2) (layer "B.Cu") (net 9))
 (segment (start 50.8 61.595) (end 50.8 74.295) (width 0.2) (layer "B.Cu") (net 9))
 (segment (start 67.19 73.78) (end 60.96 80.01) (width 0.2) (layer "B.Cu") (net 17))
 (segment (start 68.58 53.975) (end 67.19 55.365) (width 0.2) (layer "B.Cu") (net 17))
 (segment (start 67.19 55.365) (end 67.19 73.78) (width 0.2) (layer "B.Cu") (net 17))
 (segment (start 73.66 61.595) (end 72.155 63.1) (width 0.2) (layer "B.Cu") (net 14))
 (segment (start 72.155 63.1) (end 72.155 76.435) (width 0.2) (layer "B.Cu") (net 14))
 (segment (start 72.155 76.435) (end 68.58 80.01) (width 0.2) (layer "B.Cu") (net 14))
 (segment (start 71.12 53.975) (end 69.68 55.415) (width 0.2) (layer "B.Cu") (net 16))
 (segment (start 69.68 73.83) (end 63.5 80.01) (width 0.2) (layer "B.Cu") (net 16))
 (segment (start 69.68 55.415) (end 69.68 73.83) (width 0.2) (layer "B.Cu") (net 16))
 (segment (start 71.12 64.135) (end 73.025 64.135) (width 0.2) (layer "F.Cu") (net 13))
 (via (at 73.025 64.135) (size 0.6) (drill 0.3) (layers "F.Cu" "B.Cu") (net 13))
 (via (at 71.12 64.135) (size 0.6) (drill 0.3) (layers "F.Cu" "B.Cu") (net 13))
 (segment (start 71.12 61.595) (end 71.12 62.23) (width 0.2) (layer "B.Cu") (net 13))
 (segment (start 73.025 64.135) (end 73.025 78.105) (width 0.2) (layer "B.Cu") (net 13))
 (segment (start 71.12 62.23) (end 71.12 64.135) (width 0.2) (layer "B.Cu") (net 13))
 (segment (start 73.025 78.105) (end 71.12 80.01) (width 0.2) (layer "B.Cu") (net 13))
 (segment (start 73.66 64.77) (end 69.215 64.77) (width 0.2) (layer "F.Cu") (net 12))
 (segment (start 68.58 64.135) (end 68.58 61.595) (width 0.2) (layer "F.Cu") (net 12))
 (segment (start 69.215 64.77) (end 68.58 64.135) (width 0.2) (layer "F.Cu") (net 12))
 (via (at 73.66 64.77) (size 0.6) (drill 0.3) (layers "F.Cu" "B.Cu") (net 12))
 (segment (start 73.66 64.77) (end 73.66 80.01) (width 0.2) (layer "B.Cu") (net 12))
 (segment (start 42.07 78.9) (end 43.18 80.01) (width 0.2) (layer "B.Cu") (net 24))
 (segment (start 42.07 55.085) (end 42.07 78.9) (width 0.2) (layer "B.Cu") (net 24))
 (segment (start 43.18 53.975) (end 42.07 55.085) (width 0.2) (layer "B.Cu") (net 24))
 (segment (start 66.04 62.865) (end 68.58 65.405) (width 0.2) (layer "F.Cu") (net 11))
 (segment (start 66.04 61.595) (end 66.04 62.865) (width 0.2) (layer "F.Cu") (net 11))
 (segment (start 68.58 65.405) (end 76.2 65.405) (width 0.2) (layer "F.Cu") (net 11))
 (via (at 76.2 65.405) (size 0.6) (drill 0.3) (layers "F.Cu" "B.Cu") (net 11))
 (segment (start 76.2 65.405) (end 76.2 80.01) (width 0.2) (layer "B.Cu") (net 11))
 (segment (start 45.72 53.975) (end 44.62 55.075) (width 0.2) (layer "B.Cu") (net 23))
 (segment (start 44.62 55.075) (end 44.62 78.91) (width 0.2) (layer "B.Cu") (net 23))
 (segment (start 44.62 78.91) (end 45.72 80.01) (width 0.2) (layer "B.Cu") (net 23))
 (segment (start 71.755 62.515635) (end 71.755 73.66) (width 0.2) (layer "B.Cu") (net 15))
 (segment (start 71.755 73.66) (end 66.04 79.375) (width 0.2) (layer "B.Cu") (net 15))
 (segment (start 66.04 79.375) (end 66.04 80.01) (width 0.2) (layer "B.Cu") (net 15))
 (segment (start 72.39 61.880635) (end 71.755 62.515635) (width 0.2) (layer "B.Cu") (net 15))
 (segment (start 73.66 53.975) (end 72.39 55.245) (width 0.2) (layer "B.Cu") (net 15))
 (segment (start 72.39 55.245) (end 72.39 61.880635) (width 0.2) (layer "B.Cu") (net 15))
 (segment (start 62.19 61.009365) (end 62.19 76.24) (width 0.2) (layer "B.Cu") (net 18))
 (segment (start 62.19 76.24) (end 58.42 80.01) (width 0.2) (layer "B.Cu") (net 18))
 (segment (start 66.04 53.975) (end 66.04 57.159365) (width 0.2) (layer "B.Cu") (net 18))
 (segment (start 66.04 57.159365) (end 62.19 61.009365) (width 0.2) (layer "B.Cu") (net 18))
 (segment (start 53.34 73.66) (end 78.74 73.66) (width 0.2) (layer "F.Cu") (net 10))
 (via (at 53.34 73.66) (size 0.6) (drill 0.3) (layers "F.Cu" "B.Cu") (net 10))
 (via (at 78.74 73.66) (size 0.6) (drill 0.3) (layers "F.Cu" "B.Cu") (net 10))
 (segment (start 78.74 73.66) (end 78.74 80.01) (width 0.2) (layer "B.Cu") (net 10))
 (segment (start 53.34 62.23) (end 53.34 73.66) (width 0.2) (layer "B.Cu") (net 10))
 (segment (start 53.34 61.595) (end 53.34 62.23) (width 0.2) (layer "B.Cu") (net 10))
 (segment (start 54.44 78.91) (end 53.34 80.01) (width 0.2) (layer "B.Cu") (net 20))
 (segment (start 54.44 55.075) (end 54.44 78.91) (width 0.2) (layer "B.Cu") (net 20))
 (segment (start 53.34 53.975) (end 54.44 55.075) (width 0.2) (layer "B.Cu") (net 20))
 (segment (start 61.04 61.675) (end 60.96 61.595) (width 0.2) (layer "B.Cu") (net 28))
 (segment (start 61.04 64.77) (end 61.04 61.675) (width 0.2) (layer "B.Cu") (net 28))
 (segment (start 66.04 64.135) (end 63.5 61.595) (width 0.2) (layer "B.Cu") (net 27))
 (segment (start 66.04 64.77) (end 66.04 64.135) (width 0.2) (layer "B.Cu") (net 27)))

